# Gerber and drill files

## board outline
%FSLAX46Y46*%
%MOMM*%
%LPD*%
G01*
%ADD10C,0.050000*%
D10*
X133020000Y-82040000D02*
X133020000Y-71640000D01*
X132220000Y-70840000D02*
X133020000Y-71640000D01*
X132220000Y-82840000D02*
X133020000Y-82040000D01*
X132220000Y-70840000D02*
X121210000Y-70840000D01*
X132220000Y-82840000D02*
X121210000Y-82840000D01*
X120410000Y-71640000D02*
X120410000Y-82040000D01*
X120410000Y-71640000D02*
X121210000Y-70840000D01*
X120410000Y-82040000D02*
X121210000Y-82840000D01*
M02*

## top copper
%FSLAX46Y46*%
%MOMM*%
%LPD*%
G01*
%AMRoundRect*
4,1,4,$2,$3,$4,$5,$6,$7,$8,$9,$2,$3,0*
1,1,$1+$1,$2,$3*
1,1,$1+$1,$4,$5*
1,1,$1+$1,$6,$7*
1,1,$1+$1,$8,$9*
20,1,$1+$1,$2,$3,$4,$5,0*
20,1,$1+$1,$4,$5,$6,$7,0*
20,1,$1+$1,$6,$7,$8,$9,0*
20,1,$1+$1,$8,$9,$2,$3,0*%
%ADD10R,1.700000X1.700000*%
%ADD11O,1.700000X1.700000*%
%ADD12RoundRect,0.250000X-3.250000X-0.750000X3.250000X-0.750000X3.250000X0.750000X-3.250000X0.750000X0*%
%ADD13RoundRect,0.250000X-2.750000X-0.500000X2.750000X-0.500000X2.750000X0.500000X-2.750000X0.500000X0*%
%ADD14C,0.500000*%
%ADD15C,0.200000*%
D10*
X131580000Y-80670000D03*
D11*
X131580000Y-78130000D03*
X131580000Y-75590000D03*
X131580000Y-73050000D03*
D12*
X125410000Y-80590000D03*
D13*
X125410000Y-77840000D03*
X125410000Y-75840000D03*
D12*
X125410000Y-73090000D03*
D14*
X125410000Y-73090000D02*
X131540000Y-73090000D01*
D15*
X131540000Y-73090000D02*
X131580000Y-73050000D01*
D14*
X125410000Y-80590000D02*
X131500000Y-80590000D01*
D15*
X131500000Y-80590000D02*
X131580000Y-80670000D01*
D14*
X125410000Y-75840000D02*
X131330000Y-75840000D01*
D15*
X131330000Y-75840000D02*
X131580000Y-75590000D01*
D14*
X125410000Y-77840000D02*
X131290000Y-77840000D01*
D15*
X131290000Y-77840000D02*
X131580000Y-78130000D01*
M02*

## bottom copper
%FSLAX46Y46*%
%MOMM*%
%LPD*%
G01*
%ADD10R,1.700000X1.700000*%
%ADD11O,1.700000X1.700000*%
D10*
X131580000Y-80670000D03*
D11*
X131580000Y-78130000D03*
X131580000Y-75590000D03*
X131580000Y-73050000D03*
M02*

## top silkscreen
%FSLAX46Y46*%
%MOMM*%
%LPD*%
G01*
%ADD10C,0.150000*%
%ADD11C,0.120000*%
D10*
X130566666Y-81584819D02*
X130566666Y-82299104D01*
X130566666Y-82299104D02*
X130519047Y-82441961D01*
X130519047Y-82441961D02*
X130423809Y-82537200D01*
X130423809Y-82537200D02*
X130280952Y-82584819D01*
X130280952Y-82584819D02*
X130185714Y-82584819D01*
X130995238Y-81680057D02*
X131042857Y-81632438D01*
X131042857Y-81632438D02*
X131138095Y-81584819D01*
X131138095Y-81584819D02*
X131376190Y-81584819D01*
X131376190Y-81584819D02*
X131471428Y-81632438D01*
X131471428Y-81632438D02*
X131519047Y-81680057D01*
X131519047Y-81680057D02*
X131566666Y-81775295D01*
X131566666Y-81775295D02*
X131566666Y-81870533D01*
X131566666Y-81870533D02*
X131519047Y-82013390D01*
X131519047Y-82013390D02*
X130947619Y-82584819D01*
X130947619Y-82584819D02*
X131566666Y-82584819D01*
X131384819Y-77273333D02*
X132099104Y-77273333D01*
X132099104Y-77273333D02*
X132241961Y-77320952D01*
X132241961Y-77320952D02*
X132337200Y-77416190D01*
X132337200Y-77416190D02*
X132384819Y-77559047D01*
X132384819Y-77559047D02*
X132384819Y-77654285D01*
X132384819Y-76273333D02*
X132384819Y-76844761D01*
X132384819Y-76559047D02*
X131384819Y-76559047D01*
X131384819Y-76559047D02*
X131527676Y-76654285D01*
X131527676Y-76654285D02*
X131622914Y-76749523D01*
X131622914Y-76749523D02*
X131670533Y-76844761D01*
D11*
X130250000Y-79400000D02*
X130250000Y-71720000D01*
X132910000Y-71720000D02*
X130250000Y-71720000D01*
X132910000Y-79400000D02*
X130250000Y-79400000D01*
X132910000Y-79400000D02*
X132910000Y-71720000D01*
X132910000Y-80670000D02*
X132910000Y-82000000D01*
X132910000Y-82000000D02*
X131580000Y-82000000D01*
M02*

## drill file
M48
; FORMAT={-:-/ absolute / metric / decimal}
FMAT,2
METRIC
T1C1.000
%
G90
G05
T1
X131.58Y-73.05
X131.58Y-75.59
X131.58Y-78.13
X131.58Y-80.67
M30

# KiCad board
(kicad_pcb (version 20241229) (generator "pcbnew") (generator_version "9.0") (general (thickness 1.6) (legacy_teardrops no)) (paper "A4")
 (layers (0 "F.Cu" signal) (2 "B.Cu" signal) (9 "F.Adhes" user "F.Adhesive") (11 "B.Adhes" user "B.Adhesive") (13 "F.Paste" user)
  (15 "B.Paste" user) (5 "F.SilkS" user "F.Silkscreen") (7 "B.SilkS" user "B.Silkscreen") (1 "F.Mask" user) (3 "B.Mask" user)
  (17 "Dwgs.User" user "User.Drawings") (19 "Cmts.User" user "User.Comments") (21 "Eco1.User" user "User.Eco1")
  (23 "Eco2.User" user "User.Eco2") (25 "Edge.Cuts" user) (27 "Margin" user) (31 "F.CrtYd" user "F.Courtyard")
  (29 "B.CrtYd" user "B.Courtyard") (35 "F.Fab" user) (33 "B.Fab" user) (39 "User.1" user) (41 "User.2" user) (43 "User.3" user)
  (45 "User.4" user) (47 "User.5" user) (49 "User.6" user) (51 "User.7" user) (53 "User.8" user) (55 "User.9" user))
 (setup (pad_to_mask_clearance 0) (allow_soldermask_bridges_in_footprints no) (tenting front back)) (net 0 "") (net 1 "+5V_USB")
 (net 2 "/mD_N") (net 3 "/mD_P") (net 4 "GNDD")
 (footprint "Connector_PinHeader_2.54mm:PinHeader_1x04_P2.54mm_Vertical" (layer "F.Cu") (at 131.58 80.67 180)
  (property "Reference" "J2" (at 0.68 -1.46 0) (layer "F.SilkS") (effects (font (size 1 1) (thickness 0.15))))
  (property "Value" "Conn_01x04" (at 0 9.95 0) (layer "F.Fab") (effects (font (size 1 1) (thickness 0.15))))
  (fp_line (start 1.33 1.27) (end 1.33 8.95) (stroke (width 0.12) (type solid)) (layer "F.SilkS"))
  (fp_line (start -1.33 8.95) (end 1.33 8.95) (stroke (width 0.12) (type solid)) (layer "F.SilkS"))
  (fp_line (start -1.33 1.27) (end 1.33 1.27) (stroke (width 0.12) (type solid)) (layer "F.SilkS"))
  (fp_line (start -1.33 1.27) (end -1.33 8.95) (stroke (width 0.12) (type solid)) (layer "F.SilkS"))
  (fp_line (start -1.33 0) (end -1.33 -1.33) (stroke (width 0.12) (type solid)) (layer "F.SilkS"))
  (fp_line (start -1.33 -1.33) (end 0 -1.33) (stroke (width 0.12) (type solid)) (layer "F.SilkS"))
  (pad "1" thru_hole rect (at 0 0 180) (size 1.7 1.7) (drill 1) (layers "*.Cu" "*.Mask") (remove_unused_layers no) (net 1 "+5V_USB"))
  (pad "2" thru_hole oval (at 0 2.54 180) (size 1.7 1.7) (drill 1) (layers "*.Cu" "*.Mask") (remove_unused_layers no) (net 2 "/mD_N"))
  (pad "3" thru_hole oval (at 0 5.08 180) (size 1.7 1.7) (drill 1) (layers "*.Cu" "*.Mask") (remove_unused_layers no) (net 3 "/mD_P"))
  (pad "4" thru_hole oval (at 0 7.62 180) (size 1.7 1.7) (drill 1) (layers "*.Cu" "*.Mask") (remove_unused_layers no) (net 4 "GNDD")))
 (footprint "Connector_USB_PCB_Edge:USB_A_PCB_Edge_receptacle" (layer "F.Cu") (at 125.41 76.84)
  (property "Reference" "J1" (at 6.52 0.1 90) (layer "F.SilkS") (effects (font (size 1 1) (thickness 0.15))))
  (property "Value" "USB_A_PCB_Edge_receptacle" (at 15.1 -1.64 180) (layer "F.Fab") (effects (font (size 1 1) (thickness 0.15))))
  (fp_line (start -5 -5.2) (end -5 5.2) (stroke (width 0.05) (type default)) (layer "Edge.Cuts"))
  (fp_line (start -5 -5.2) (end -4.2 -6) (stroke (width 0.05) (type default)) (layer "Edge.Cuts"))
  (fp_line (start -5 5.2) (end -4.2 6) (stroke (width 0.05) (type default)) (layer "Edge.Cuts"))
  (pad "1" smd roundrect (at 0 3.75) (size 7 2) (layers "F.Cu" "F.Mask" "F.Paste") (roundrect_rratio 0.125) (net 1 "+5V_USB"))
  (pad "2" smd roundrect (at 0 1) (size 6 1.5) (layers "F.Cu" "F.Mask" "F.Paste") (roundrect_rratio 0.1666666667) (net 2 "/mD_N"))
  (pad "3" smd roundrect (at 0 -1) (size 6 1.5) (layers "F.Cu" "F.Mask" "F.Paste") (roundrect_rratio 0.1666666667) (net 3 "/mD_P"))
  (pad "4" smd roundrect (at 0 -3.75) (size 7 2) (layers "F.Cu" "F.Mask" "F.Paste") (roundrect_rratio 0.125) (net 4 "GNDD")))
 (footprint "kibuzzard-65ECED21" (layer "B.Cu") (at 128.0759 78.20576)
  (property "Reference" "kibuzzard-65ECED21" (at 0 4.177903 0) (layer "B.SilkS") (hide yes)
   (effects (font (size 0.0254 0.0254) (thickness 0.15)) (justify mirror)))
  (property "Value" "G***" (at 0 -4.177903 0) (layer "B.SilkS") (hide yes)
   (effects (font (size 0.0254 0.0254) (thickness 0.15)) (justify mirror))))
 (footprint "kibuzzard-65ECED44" (layer "B.Cu") (at 127.0859 73.04576)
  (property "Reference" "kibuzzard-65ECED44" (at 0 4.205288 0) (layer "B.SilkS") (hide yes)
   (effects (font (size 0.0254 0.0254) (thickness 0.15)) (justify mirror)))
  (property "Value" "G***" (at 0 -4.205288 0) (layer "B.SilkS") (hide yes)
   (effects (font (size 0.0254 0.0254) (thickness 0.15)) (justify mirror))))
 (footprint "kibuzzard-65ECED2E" (layer "B.Cu") (at 128.1659 75.62576)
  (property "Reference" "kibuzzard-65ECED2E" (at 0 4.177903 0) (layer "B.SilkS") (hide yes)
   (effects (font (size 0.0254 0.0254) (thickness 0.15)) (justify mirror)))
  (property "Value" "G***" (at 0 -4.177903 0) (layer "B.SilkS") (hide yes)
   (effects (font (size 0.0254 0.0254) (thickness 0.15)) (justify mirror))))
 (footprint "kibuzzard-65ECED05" (layer "B.Cu") (at 127.3359 80.86576)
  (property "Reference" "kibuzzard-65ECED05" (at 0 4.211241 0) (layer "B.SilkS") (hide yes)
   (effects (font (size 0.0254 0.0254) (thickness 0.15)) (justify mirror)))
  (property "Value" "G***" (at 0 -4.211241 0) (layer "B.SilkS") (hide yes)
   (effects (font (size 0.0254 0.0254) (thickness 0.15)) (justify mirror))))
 (gr_line (start 133.02 82.04) (end 133.02 71.64) (stroke (width 0.05) (type default)) (layer "Edge.Cuts"))
 (gr_line (start 132.22 70.84) (end 133.02 71.64) (stroke (width 0.05) (type default)) (layer "Edge.Cuts"))
 (gr_line (start 132.22 82.84) (end 133.02 82.04) (stroke (width 0.05) (type default)) (layer "Edge.Cuts"))
 (gr_line (start 132.22 70.84) (end 121.21 70.84) (stroke (width 0.05) (type default)) (layer "Edge.Cuts"))
 (gr_line (start 132.22 82.84) (end 121.21 82.84) (stroke (width 0.05) (type default)) (layer "Edge.Cuts"))
 (segment (start 125.41 73.09) (end 131.54 73.09) (width 0.5) (layer "F.Cu") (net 4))
 (segment (start 131.54 73.09) (end 131.58 73.05) (width 0.2) (layer "F.Cu") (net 4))
 (segment (start 125.41 80.59) (end 131.5 80.59) (width 0.5) (layer "F.Cu") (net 1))
 (segment (start 131.5 80.59) (end 131.58 80.67) (width 0.2) (layer "F.Cu") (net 1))
 (segment (start 125.41 75.84) (end 131.33 75.84) (width 0.5) (layer "F.Cu") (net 3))
 (segment (start 131.33 75.84) (end 131.58 75.59) (width 0.2) (layer "F.Cu") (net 3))
 (segment (start 125.41 77.84) (end 131.29 77.84) (width 0.5) (layer "F.Cu") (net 2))
 (segment (start 131.29 77.84) (end 131.58 78.13) (width 0.2) (layer "F.Cu") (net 2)))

